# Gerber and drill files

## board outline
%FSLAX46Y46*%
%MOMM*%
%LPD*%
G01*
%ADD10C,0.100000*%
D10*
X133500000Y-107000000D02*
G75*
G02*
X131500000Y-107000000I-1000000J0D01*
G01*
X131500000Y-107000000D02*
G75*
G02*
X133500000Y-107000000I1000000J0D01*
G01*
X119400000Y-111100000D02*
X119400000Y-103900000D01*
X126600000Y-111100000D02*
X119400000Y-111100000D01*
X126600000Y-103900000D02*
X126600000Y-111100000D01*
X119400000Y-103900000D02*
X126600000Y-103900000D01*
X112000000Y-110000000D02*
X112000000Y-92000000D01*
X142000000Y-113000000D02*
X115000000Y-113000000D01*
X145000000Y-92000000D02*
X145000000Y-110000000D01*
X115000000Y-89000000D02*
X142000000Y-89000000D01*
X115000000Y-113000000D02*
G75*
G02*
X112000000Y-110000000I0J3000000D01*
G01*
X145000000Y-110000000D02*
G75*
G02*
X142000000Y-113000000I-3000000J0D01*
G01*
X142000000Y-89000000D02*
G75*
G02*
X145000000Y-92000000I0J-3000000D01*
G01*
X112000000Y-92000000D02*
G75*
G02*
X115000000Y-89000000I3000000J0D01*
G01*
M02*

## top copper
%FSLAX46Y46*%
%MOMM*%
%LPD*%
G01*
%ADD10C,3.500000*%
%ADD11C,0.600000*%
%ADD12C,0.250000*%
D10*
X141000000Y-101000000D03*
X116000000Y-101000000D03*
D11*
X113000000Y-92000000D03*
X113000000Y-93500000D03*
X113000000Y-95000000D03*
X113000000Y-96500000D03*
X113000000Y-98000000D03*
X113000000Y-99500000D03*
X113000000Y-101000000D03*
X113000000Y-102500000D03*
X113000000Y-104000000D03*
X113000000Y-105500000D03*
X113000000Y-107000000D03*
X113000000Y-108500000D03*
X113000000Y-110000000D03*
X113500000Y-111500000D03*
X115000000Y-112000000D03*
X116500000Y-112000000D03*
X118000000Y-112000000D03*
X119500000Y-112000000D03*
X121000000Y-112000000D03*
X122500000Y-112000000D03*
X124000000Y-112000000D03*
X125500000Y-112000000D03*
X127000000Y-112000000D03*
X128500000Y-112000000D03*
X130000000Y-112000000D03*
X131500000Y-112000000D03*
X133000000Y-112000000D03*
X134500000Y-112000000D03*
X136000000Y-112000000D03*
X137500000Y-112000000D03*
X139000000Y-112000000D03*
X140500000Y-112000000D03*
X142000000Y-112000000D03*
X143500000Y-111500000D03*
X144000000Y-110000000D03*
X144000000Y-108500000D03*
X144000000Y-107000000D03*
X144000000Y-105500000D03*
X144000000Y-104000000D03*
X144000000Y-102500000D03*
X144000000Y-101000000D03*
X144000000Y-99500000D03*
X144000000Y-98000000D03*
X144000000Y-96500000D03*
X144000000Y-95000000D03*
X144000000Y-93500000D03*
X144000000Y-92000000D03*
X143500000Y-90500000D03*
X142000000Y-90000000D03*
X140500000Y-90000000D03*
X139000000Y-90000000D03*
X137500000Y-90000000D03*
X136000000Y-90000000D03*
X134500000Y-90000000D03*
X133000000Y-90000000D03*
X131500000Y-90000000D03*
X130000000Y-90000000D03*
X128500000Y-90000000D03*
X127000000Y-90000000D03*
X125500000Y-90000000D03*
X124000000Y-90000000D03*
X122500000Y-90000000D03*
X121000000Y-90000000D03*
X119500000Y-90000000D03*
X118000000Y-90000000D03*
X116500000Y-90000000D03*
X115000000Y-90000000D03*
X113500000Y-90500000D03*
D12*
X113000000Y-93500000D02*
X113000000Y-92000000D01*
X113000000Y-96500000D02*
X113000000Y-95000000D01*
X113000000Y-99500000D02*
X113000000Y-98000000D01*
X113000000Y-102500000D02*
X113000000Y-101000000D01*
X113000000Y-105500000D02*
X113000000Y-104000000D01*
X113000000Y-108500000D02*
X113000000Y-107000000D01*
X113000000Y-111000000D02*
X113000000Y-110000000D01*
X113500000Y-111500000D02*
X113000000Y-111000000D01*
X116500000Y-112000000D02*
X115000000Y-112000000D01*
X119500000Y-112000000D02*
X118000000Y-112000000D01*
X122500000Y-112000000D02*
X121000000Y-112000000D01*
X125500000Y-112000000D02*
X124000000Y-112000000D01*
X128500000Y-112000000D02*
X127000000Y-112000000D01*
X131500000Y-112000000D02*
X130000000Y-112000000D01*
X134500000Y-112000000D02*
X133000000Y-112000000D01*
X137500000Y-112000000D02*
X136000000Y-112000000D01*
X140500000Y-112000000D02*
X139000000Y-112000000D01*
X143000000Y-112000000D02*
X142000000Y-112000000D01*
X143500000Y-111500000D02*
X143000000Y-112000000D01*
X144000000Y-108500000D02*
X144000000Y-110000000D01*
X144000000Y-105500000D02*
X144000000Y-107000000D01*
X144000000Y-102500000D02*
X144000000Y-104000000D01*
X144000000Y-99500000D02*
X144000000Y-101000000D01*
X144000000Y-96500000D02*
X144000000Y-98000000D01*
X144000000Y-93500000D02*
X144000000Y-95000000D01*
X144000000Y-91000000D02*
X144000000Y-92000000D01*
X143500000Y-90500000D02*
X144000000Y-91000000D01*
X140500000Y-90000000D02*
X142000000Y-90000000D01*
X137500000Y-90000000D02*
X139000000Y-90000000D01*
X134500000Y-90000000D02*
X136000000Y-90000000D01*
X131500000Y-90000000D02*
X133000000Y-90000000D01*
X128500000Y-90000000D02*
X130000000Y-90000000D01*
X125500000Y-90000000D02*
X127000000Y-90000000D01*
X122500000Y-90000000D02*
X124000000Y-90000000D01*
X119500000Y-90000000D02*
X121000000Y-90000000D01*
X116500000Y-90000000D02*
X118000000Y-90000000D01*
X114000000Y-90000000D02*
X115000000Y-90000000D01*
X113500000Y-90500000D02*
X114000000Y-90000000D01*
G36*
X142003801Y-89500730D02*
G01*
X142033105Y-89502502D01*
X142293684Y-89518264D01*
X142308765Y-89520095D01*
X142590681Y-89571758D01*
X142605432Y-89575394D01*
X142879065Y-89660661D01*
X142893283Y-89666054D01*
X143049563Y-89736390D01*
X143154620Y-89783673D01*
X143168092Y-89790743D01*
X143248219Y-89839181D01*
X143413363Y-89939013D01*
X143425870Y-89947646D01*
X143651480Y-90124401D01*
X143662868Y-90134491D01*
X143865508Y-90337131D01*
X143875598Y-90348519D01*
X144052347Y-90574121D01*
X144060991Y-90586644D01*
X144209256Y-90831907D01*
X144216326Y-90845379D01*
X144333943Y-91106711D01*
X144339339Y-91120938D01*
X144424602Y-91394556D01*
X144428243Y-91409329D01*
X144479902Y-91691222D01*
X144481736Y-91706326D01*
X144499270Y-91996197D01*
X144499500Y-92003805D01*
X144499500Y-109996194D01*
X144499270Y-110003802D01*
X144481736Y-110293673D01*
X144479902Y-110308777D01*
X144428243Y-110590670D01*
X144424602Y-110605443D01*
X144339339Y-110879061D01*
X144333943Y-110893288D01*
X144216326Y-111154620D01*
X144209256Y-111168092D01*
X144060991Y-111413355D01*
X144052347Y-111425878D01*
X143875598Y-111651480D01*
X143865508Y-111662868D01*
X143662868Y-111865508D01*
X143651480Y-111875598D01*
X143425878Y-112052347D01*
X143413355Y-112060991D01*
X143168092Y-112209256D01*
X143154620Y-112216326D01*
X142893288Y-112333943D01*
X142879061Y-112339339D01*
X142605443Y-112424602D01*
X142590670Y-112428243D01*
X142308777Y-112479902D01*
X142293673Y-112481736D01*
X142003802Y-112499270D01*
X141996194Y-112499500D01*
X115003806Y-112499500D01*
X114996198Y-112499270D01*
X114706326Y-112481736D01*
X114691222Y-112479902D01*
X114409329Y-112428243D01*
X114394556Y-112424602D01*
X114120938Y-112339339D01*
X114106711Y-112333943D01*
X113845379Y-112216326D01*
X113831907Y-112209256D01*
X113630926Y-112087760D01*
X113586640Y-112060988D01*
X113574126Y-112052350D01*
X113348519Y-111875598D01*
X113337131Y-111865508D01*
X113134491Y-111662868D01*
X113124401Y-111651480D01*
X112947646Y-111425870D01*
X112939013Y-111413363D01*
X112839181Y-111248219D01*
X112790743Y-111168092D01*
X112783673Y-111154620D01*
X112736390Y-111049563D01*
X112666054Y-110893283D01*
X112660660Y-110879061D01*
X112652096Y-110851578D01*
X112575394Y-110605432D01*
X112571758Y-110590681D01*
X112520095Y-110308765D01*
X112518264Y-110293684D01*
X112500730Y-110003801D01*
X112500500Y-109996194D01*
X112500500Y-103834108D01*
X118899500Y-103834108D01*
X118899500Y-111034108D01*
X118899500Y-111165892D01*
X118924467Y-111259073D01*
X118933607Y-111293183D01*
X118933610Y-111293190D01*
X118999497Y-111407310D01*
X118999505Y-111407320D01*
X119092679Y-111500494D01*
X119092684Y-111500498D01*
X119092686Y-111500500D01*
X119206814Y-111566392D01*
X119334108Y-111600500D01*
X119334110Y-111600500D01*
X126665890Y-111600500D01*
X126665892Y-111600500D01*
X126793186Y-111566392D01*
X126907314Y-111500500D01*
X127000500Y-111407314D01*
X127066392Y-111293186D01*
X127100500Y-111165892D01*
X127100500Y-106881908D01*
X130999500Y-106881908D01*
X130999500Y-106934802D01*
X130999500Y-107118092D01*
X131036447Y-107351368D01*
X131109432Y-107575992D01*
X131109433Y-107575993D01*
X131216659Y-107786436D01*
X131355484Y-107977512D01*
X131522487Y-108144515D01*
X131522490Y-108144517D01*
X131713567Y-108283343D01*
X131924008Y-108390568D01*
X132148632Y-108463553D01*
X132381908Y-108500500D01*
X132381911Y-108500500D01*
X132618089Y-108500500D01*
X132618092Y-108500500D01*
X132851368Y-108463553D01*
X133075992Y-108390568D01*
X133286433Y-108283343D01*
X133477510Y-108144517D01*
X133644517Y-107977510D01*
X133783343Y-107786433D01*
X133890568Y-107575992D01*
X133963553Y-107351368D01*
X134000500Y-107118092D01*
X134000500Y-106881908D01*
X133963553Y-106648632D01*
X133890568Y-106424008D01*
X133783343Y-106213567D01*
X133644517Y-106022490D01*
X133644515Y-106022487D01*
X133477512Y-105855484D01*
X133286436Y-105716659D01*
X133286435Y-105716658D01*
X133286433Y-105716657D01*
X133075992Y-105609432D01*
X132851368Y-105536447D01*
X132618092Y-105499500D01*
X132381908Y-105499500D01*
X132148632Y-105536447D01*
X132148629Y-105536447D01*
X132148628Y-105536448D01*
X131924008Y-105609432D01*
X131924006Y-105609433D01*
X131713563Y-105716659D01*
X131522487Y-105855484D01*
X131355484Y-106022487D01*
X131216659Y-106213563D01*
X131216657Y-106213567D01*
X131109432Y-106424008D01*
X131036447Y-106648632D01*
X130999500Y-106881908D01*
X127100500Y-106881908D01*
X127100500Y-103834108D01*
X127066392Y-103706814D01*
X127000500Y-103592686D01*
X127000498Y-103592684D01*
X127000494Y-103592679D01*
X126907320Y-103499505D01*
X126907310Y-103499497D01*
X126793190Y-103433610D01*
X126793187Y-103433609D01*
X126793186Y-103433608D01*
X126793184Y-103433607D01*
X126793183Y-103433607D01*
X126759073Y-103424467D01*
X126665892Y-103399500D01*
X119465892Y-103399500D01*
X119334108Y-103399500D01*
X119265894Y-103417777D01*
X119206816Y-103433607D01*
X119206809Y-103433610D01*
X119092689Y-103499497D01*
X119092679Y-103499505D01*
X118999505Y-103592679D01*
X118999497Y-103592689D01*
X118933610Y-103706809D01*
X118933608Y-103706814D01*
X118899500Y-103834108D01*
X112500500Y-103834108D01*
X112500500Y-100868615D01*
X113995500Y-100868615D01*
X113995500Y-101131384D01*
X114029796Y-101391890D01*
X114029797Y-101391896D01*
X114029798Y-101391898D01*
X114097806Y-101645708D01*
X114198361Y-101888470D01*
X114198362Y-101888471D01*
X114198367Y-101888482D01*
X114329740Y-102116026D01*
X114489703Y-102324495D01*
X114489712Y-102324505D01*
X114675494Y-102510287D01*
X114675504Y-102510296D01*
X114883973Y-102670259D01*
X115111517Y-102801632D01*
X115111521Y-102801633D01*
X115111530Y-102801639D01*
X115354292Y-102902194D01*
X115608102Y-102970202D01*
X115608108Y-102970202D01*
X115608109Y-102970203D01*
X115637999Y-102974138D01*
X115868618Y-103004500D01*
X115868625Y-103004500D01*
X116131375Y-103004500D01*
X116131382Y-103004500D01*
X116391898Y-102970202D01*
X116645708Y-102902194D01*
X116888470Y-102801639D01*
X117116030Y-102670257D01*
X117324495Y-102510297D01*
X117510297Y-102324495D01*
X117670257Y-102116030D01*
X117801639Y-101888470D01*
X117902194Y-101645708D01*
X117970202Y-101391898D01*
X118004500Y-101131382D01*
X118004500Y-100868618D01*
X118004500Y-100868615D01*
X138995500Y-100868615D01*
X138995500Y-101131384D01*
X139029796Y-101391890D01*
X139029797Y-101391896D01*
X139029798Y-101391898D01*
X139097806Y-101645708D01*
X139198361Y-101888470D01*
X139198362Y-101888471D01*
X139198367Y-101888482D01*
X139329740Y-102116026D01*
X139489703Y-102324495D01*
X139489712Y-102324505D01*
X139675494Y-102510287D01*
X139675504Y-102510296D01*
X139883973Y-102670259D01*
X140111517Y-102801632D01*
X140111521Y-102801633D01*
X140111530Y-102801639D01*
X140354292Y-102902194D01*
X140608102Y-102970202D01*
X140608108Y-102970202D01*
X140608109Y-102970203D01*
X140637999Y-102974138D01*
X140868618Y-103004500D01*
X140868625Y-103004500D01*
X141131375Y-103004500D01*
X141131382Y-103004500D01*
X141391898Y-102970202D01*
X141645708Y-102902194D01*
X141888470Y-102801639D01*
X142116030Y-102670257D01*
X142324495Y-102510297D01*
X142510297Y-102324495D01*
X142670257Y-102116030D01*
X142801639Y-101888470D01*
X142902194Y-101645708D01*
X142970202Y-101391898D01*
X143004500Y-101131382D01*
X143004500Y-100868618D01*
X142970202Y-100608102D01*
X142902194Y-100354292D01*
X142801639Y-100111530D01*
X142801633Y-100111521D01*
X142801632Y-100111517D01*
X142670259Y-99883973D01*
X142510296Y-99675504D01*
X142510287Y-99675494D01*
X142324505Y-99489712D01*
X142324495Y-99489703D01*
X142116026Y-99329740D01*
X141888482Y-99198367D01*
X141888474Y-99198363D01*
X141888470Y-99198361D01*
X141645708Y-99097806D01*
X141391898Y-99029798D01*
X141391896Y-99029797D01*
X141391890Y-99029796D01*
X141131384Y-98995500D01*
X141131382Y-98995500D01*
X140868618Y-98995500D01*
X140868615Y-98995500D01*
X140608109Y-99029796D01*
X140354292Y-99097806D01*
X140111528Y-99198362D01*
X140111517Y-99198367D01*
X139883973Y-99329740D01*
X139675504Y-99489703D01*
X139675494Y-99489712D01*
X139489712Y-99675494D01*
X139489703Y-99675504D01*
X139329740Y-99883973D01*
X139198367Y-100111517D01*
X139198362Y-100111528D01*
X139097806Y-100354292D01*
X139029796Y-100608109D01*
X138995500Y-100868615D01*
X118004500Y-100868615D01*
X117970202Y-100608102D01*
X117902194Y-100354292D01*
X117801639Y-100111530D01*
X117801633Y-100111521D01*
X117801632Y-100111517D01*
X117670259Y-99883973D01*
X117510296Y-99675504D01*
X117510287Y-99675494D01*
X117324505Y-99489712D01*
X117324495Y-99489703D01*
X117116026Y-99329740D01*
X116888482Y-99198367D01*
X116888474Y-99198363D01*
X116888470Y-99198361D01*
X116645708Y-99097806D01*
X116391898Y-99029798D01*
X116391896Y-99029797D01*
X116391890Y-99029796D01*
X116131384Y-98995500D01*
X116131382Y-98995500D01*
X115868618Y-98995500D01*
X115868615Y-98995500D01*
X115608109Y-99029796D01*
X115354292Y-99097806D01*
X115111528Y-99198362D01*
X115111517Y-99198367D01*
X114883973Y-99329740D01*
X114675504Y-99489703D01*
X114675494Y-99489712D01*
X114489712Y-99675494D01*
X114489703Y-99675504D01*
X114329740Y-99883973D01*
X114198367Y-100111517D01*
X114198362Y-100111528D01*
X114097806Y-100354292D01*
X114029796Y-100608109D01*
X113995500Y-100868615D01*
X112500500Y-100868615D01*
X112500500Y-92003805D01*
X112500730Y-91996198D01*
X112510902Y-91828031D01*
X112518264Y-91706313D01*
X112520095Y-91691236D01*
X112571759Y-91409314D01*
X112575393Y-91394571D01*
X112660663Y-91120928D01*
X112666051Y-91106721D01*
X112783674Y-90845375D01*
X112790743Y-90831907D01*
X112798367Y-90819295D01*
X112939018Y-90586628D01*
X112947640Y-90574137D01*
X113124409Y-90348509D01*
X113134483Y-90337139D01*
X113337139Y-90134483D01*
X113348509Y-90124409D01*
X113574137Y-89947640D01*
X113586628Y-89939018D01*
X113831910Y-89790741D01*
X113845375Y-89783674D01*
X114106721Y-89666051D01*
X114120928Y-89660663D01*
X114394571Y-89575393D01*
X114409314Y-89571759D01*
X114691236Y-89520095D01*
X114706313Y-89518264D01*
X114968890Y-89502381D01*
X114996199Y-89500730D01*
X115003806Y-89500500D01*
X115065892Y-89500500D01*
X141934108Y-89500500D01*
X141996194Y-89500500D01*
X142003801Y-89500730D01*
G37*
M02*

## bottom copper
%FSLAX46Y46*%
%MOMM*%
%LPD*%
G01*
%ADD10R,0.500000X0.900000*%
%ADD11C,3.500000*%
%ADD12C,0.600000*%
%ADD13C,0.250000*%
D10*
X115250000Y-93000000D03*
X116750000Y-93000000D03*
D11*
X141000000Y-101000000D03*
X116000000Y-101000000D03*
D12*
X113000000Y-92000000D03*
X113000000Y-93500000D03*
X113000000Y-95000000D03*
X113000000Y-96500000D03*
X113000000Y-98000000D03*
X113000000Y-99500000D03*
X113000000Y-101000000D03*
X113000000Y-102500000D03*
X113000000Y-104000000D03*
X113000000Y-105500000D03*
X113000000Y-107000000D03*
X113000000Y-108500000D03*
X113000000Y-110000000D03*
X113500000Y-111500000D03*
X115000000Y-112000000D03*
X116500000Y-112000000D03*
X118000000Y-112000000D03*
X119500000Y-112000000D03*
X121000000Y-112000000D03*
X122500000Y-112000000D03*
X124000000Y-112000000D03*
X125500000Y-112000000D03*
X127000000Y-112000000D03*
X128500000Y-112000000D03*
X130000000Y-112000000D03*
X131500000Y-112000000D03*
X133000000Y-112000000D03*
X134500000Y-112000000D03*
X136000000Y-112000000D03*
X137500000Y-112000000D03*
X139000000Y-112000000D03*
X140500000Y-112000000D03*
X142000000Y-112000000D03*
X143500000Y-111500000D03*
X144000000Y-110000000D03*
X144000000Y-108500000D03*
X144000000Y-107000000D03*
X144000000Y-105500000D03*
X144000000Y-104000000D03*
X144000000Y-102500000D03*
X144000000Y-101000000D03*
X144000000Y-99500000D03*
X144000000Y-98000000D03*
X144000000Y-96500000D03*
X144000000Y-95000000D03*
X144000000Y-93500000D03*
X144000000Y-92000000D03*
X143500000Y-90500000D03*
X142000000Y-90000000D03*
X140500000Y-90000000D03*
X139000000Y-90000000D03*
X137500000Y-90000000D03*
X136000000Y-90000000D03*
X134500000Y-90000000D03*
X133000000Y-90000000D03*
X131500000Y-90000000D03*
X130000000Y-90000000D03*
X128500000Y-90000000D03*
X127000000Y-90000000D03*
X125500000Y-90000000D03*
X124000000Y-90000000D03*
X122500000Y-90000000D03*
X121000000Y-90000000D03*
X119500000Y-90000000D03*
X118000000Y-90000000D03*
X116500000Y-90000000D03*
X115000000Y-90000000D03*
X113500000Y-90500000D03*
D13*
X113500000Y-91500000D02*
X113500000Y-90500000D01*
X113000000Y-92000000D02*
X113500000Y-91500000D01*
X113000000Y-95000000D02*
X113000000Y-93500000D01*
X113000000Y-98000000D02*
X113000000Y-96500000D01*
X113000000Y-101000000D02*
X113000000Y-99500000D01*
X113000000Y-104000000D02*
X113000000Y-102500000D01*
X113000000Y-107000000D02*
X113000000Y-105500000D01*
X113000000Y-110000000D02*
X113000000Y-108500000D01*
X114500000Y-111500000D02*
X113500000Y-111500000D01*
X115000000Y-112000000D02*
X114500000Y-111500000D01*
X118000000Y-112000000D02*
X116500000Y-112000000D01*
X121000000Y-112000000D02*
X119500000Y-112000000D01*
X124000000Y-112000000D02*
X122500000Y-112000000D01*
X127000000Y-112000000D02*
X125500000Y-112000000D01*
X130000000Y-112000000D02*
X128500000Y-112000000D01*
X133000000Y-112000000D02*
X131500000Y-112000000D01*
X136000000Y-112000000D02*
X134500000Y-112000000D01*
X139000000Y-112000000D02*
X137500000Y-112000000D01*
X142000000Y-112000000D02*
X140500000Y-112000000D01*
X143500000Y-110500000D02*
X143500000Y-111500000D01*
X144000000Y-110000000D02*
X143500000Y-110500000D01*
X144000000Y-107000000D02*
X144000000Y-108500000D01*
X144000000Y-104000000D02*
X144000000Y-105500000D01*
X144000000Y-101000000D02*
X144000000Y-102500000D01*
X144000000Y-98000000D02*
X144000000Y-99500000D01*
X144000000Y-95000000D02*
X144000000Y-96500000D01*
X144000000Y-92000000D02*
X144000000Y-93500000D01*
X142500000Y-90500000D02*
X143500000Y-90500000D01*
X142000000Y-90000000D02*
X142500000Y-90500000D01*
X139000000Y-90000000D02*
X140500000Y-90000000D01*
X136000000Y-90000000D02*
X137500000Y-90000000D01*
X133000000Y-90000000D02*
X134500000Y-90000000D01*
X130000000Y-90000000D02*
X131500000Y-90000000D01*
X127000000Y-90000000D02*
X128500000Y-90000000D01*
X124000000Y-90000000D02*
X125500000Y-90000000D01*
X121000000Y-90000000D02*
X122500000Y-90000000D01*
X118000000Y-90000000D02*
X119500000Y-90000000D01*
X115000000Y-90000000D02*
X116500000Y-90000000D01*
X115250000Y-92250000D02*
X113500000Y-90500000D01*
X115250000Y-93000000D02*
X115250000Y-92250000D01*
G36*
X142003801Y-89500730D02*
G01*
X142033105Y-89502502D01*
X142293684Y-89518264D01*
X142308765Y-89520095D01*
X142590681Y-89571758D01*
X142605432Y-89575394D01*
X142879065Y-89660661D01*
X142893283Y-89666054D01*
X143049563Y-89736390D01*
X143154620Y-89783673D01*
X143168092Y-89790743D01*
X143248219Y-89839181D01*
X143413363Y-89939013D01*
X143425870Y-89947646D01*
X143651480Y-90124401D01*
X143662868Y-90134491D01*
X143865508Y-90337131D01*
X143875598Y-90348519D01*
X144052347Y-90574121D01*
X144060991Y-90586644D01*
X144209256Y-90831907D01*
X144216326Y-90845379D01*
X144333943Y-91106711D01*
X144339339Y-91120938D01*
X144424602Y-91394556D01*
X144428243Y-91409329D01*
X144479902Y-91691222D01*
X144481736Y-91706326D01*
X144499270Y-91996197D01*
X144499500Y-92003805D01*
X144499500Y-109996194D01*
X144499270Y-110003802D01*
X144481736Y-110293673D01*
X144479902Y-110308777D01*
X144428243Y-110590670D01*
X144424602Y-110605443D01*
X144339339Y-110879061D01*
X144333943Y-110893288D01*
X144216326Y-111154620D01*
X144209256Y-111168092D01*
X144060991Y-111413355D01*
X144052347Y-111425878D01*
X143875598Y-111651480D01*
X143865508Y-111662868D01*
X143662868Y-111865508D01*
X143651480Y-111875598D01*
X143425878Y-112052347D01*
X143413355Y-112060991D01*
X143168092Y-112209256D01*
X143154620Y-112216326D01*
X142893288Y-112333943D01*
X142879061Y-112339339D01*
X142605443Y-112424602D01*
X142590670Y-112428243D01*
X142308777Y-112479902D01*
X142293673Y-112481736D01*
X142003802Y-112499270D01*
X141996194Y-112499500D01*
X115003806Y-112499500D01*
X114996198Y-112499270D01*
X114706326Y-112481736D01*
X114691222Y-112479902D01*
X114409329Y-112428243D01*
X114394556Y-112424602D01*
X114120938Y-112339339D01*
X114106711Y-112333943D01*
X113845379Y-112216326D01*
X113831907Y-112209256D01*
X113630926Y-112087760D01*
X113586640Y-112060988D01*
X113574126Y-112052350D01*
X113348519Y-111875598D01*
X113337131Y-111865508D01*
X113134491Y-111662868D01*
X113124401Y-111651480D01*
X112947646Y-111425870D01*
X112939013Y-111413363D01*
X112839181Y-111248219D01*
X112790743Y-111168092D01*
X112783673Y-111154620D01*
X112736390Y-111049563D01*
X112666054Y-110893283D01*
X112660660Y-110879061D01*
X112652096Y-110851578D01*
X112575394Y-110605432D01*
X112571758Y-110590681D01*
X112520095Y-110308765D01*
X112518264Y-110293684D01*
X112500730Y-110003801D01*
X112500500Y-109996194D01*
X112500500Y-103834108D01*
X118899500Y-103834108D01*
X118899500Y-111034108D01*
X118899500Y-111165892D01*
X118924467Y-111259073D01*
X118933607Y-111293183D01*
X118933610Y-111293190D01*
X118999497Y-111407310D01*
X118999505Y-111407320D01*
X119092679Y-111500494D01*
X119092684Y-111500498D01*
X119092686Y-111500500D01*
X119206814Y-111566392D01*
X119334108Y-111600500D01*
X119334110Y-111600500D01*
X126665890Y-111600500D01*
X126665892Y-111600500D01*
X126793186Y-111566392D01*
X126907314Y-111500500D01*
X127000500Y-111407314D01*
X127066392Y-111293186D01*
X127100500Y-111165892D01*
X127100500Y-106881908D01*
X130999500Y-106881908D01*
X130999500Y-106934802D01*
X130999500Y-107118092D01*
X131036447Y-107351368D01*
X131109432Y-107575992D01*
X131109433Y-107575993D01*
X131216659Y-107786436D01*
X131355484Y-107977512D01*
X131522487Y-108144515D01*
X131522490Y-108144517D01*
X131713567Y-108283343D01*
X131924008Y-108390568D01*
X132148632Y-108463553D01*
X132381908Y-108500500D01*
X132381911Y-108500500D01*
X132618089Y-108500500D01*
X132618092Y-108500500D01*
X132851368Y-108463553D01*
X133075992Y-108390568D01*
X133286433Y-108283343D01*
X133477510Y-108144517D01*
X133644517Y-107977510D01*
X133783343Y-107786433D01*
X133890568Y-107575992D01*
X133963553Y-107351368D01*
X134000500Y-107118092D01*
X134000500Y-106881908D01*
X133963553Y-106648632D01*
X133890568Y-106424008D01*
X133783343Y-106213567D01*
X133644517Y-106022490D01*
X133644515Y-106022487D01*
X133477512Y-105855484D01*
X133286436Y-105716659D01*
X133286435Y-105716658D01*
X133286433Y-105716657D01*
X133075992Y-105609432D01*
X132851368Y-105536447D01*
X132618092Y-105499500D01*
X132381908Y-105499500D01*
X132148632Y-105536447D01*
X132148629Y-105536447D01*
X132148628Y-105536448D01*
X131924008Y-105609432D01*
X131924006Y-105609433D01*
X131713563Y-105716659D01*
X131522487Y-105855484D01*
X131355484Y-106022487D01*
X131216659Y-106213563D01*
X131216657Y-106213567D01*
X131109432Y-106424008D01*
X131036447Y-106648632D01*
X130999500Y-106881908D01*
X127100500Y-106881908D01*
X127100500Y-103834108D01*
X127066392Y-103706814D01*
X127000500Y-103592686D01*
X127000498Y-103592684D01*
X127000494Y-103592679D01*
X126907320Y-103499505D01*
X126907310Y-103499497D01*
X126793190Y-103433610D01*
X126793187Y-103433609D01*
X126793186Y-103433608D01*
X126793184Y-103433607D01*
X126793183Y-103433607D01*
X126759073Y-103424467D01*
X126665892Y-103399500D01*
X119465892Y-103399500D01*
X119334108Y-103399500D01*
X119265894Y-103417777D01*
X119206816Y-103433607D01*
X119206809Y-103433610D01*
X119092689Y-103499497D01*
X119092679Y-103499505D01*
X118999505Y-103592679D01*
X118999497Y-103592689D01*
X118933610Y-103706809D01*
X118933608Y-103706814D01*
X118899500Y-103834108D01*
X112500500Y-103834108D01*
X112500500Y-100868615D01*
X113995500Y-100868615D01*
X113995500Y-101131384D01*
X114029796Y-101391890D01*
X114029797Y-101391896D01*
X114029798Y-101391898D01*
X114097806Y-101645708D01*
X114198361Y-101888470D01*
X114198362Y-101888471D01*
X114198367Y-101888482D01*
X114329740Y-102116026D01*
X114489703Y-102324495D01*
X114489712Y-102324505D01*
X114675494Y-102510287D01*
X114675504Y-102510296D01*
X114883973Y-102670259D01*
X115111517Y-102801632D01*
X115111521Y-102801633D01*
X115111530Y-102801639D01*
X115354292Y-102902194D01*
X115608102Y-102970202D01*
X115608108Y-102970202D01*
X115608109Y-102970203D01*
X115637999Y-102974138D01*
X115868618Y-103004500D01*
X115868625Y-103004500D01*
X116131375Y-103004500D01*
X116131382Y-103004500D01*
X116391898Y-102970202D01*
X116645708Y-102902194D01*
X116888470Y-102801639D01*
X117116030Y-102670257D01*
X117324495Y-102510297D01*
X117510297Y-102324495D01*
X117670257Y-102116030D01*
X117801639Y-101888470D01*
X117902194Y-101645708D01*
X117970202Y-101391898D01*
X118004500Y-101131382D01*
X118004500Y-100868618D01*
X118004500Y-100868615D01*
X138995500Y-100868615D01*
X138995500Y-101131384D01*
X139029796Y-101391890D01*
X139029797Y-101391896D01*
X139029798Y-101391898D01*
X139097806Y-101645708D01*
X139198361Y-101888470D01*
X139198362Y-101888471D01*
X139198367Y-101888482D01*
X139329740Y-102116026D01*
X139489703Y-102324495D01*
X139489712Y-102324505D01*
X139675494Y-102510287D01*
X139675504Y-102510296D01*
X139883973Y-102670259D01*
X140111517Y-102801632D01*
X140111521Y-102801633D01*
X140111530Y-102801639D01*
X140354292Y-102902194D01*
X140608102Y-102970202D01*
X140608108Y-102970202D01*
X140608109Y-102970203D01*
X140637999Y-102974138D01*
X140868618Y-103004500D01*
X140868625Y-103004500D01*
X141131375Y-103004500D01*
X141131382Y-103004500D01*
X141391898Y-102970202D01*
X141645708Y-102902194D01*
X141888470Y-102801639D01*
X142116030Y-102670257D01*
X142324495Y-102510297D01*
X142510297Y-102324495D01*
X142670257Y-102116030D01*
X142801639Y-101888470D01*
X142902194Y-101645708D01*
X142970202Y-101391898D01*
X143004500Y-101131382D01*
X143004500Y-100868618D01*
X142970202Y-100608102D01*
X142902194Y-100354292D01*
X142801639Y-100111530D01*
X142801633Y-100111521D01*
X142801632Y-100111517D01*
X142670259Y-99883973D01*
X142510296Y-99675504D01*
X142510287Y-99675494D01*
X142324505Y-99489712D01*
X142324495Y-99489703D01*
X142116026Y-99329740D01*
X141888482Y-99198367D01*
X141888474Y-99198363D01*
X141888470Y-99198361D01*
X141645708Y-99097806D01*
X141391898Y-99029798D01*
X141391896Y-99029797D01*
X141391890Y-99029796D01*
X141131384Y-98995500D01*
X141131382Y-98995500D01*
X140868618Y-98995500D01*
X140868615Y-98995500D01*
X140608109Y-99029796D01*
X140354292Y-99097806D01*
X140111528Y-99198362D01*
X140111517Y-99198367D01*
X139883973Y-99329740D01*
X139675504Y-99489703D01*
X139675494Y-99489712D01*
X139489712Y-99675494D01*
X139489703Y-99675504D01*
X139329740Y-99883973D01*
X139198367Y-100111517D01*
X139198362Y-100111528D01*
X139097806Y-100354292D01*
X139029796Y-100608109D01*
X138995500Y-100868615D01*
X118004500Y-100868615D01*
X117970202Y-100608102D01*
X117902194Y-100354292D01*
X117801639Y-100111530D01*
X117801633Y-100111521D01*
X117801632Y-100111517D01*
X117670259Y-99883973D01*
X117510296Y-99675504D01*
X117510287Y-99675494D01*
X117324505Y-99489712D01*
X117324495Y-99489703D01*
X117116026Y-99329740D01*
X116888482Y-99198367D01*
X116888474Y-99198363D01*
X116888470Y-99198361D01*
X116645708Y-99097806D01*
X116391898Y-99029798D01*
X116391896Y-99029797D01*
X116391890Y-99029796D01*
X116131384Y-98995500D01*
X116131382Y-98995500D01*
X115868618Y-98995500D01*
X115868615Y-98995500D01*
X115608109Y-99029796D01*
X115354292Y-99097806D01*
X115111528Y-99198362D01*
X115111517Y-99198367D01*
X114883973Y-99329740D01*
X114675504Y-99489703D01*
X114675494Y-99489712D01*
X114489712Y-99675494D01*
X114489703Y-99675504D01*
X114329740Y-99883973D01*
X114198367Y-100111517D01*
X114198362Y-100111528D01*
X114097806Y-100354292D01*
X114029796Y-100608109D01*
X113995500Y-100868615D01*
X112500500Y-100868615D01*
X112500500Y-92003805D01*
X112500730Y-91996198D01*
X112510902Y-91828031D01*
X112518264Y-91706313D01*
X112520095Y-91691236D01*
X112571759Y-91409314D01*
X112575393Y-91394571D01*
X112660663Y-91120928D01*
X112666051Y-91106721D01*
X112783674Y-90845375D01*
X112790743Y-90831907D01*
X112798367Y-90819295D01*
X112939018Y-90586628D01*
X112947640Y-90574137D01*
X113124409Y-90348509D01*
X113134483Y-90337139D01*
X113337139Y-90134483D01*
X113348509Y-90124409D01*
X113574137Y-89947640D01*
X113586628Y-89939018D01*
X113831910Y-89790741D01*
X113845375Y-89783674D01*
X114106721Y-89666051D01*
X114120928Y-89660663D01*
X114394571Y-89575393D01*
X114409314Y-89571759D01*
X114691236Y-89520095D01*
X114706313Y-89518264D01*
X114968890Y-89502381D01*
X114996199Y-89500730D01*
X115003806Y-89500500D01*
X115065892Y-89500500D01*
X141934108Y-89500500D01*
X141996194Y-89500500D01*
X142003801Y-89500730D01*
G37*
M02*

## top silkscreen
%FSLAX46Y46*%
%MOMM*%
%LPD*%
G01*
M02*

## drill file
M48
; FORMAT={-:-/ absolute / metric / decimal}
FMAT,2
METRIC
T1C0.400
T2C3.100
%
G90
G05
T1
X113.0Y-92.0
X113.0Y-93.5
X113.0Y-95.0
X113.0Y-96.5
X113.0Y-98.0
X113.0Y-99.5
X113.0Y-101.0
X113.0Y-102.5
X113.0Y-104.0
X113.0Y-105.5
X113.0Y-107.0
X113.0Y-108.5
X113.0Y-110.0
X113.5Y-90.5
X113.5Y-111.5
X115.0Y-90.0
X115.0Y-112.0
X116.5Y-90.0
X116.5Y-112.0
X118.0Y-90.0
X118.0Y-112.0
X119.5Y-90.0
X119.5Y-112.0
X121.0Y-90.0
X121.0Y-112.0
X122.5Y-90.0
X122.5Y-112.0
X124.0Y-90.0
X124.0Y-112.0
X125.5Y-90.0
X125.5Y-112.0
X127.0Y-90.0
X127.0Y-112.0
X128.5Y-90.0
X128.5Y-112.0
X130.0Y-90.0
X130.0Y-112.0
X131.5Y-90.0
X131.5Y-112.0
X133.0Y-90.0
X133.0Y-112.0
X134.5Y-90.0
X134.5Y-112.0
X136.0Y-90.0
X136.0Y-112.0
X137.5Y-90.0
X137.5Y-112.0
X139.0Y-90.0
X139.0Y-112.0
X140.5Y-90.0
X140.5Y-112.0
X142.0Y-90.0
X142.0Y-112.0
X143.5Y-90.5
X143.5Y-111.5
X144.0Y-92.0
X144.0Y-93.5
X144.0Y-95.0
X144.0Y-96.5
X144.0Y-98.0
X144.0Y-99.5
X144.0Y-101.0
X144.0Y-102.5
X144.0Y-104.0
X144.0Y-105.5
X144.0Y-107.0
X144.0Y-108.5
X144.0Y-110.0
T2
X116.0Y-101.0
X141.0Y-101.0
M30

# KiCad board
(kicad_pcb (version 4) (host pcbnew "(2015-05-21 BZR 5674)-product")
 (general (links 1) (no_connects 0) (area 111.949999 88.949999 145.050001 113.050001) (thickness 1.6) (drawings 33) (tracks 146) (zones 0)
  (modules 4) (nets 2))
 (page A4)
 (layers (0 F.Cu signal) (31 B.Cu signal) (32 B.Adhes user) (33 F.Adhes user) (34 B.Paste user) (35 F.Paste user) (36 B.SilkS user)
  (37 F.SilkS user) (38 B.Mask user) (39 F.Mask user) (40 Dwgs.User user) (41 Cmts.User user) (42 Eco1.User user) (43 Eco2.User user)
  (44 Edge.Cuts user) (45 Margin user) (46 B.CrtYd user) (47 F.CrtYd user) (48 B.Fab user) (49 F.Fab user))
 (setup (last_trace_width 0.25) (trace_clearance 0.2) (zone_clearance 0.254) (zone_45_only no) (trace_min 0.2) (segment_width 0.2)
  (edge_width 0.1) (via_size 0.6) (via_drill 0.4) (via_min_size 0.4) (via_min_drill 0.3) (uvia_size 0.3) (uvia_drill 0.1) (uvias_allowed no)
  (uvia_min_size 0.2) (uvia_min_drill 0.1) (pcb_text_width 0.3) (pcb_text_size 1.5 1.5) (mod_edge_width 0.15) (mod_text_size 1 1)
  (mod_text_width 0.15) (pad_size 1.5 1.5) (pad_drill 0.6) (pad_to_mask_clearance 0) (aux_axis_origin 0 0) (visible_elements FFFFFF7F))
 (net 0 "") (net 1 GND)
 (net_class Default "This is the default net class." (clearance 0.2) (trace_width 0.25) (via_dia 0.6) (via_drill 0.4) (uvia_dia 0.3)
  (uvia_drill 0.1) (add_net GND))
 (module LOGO (layer F.Cu) (at 123 95.25)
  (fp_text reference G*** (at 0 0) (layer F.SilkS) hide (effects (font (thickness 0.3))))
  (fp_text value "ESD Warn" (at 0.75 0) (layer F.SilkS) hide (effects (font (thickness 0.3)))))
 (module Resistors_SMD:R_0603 (layer B.Cu) (at 116 93) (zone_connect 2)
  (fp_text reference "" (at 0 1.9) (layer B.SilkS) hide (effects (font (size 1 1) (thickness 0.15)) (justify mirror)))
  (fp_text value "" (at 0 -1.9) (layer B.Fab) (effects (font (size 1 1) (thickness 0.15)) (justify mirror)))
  (pad 1 smd rect (at -0.75 0) (size 0.5 0.9) (layers B.Cu B.Paste B.Mask) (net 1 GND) (zone_connect 2))
  (pad 2 smd rect (at 0.75 0) (size 0.5 0.9) (layers B.Cu B.Paste B.Mask) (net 1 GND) (zone_connect 2)))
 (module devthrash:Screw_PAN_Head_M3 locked (layer B.Cu) (at 141 101)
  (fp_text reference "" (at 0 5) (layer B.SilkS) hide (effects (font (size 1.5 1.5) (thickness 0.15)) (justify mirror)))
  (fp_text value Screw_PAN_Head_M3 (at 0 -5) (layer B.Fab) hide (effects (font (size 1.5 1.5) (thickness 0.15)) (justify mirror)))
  (pad "" np_thru_hole circle (at 0 0) (size 3.5 3.5) (drill 3.1) (layers *.Cu *.Mask B.SilkS)))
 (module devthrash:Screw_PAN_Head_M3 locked (layer B.Cu) (at 116 101)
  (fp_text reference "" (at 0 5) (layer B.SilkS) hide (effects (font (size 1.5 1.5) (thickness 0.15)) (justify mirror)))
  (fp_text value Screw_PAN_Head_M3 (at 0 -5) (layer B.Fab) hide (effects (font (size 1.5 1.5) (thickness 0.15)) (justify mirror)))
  (pad "" np_thru_hole circle (at 0 0) (size 3.5 3.5) (drill 3.1) (layers *.Cu *.Mask B.SilkS)))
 (gr_circle (center 132.5 107) (end 133.5 107) (layer Edge.Cuts) (width 0.1))
 (gr_line (start 119.4 111.1) (end 119.4 103.9) (angle 90) (layer Edge.Cuts) (width 0.1))
 (gr_line (start 126.6 111.1) (end 119.4 111.1) (angle 90) (layer Edge.Cuts) (width 0.1))
 (gr_line (start 126.6 103.9) (end 126.6 111.1) (angle 90) (layer Edge.Cuts) (width 0.1))
 (gr_line (start 119.4 103.9) (end 126.6 103.9) (angle 90) (layer Edge.Cuts) (width 0.1))
 (gr_line (start 112 110) (end 112 92) (angle 90) (layer Edge.Cuts) (width 0.1))
 (gr_line (start 142 113) (end 115 113) (angle 90) (layer Edge.Cuts) (width 0.1))
 (gr_line (start 145 92) (end 145 110) (angle 90) (layer Edge.Cuts) (width 0.1))
 (gr_line (start 115 89) (end 142 89) (angle 90) (layer Edge.Cuts) (width 0.1))
 (gr_arc (start 115 110) (end 115 113) (angle 90) (layer Edge.Cuts) (width 0.1))
 (gr_arc (start 142 110) (end 145 110) (angle 90) (layer Edge.Cuts) (width 0.1))
 (gr_arc (start 142 92) (end 142 89) (angle 90) (layer Edge.Cuts) (width 0.1))
 (gr_arc (start 115 92) (end 112 92) (angle 90) (layer Edge.Cuts) (width 0.1))
 (segment (start 113.5 91.5) (end 113.5 90.5) (width 0.25) (layer B.Cu) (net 1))
 (segment (start 113 92) (end 113.5 91.5) (width 0.25) (layer B.Cu) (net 1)) (via (at 113 92) (size 0.6) (layers F.Cu B.Cu) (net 1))
 (segment (start 113 93.5) (end 113 92) (width 0.25) (layer F.Cu) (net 1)) (via (at 113 93.5) (size 0.6) (layers F.Cu B.Cu) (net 1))
 (segment (start 113 95) (end 113 93.5) (width 0.25) (layer B.Cu) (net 1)) (via (at 113 95) (size 0.6) (layers F.Cu B.Cu) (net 1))
 (segment (start 113 96.5) (end 113 95) (width 0.25) (layer F.Cu) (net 1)) (via (at 113 96.5) (size 0.6) (layers F.Cu B.Cu) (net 1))
 (segment (start 113 98) (end 113 96.5) (width 0.25) (layer B.Cu) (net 1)) (via (at 113 98) (size 0.6) (layers F.Cu B.Cu) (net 1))
 (segment (start 113 99.5) (end 113 98) (width 0.25) (layer F.Cu) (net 1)) (via (at 113 99.5) (size 0.6) (layers F.Cu B.Cu) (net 1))
 (segment (start 113 101) (end 113 99.5) (width 0.25) (layer B.Cu) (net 1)) (via (at 113 101) (size 0.6) (layers F.Cu B.Cu) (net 1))
 (segment (start 113 102.5) (end 113 101) (width 0.25) (layer F.Cu) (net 1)) (via (at 113 102.5) (size 0.6) (layers F.Cu B.Cu) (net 1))
 (segment (start 113 104) (end 113 102.5) (width 0.25) (layer B.Cu) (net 1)) (via (at 113 104) (size 0.6) (layers F.Cu B.Cu) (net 1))
 (segment (start 113 105.5) (end 113 104) (width 0.25) (layer F.Cu) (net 1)) (via (at 113 105.5) (size 0.6) (layers F.Cu B.Cu) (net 1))
 (segment (start 113 107) (end 113 105.5) (width 0.25) (layer B.Cu) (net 1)) (via (at 113 107) (size 0.6) (layers F.Cu B.Cu) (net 1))
 (segment (start 113 108.5) (end 113 107) (width 0.25) (layer F.Cu) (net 1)) (via (at 113 108.5) (size 0.6) (layers F.Cu B.Cu) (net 1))
 (segment (start 113 110) (end 113 108.5) (width 0.25) (layer B.Cu) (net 1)) (via (at 113 110) (size 0.6) (layers F.Cu B.Cu) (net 1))
 (segment (start 113 111) (end 113 110) (width 0.25) (layer F.Cu) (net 1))
 (segment (start 113.5 111.5) (end 113 111) (width 0.25) (layer F.Cu) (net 1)) (via (at 113.5 111.5) (size 0.6) (layers F.Cu B.Cu) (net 1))
 (segment (start 114.5 111.5) (end 113.5 111.5) (width 0.25) (layer B.Cu) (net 1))
 (segment (start 115 112) (end 114.5 111.5) (width 0.25) (layer B.Cu) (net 1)) (via (at 115 112) (size 0.6) (layers F.Cu B.Cu) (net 1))
 (segment (start 116.5 112) (end 115 112) (width 0.25) (layer F.Cu) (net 1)) (via (at 116.5 112) (size 0.6) (layers F.Cu B.Cu) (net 1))
 (segment (start 118 112) (end 116.5 112) (width 0.25) (layer B.Cu) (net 1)) (via (at 118 112) (size 0.6) (layers F.Cu B.Cu) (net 1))
 (segment (start 119.5 112) (end 118 112) (width 0.25) (layer F.Cu) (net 1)) (via (at 119.5 112) (size 0.6) (layers F.Cu B.Cu) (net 1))
 (segment (start 121 112) (end 119.5 112) (width 0.25) (layer B.Cu) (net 1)) (via (at 121 112) (size 0.6) (layers F.Cu B.Cu) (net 1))
 (segment (start 122.5 112) (end 121 112) (width 0.25) (layer F.Cu) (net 1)) (via (at 122.5 112) (size 0.6) (layers F.Cu B.Cu) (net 1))
 (segment (start 124 112) (end 122.5 112) (width 0.25) (layer B.Cu) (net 1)) (via (at 124 112) (size 0.6) (layers F.Cu B.Cu) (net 1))
 (segment (start 125.5 112) (end 124 112) (width 0.25) (layer F.Cu) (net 1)) (via (at 125.5 112) (size 0.6) (layers F.Cu B.Cu) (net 1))
 (segment (start 127 112) (end 125.5 112) (width 0.25) (layer B.Cu) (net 1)) (via (at 127 112) (size 0.6) (layers F.Cu B.Cu) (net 1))
 (segment (start 128.5 112) (end 127 112) (width 0.25) (layer F.Cu) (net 1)) (via (at 128.5 112) (size 0.6) (layers F.Cu B.Cu) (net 1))
 (segment (start 130 112) (end 128.5 112) (width 0.25) (layer B.Cu) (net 1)) (via (at 130 112) (size 0.6) (layers F.Cu B.Cu) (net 1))
 (segment (start 131.5 112) (end 130 112) (width 0.25) (layer F.Cu) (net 1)) (via (at 131.5 112) (size 0.6) (layers F.Cu B.Cu) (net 1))
 (segment (start 133 112) (end 131.5 112) (width 0.25) (layer B.Cu) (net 1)) (via (at 133 112) (size 0.6) (layers F.Cu B.Cu) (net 1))
 (segment (start 134.5 112) (end 133 112) (width 0.25) (layer F.Cu) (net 1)) (via (at 134.5 112) (size 0.6) (layers F.Cu B.Cu) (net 1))
 (segment (start 136 112) (end 134.5 112) (width 0.25) (layer B.Cu) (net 1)) (via (at 136 112) (size 0.6) (layers F.Cu B.Cu) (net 1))
 (segment (start 137.5 112) (end 136 112) (width 0.25) (layer F.Cu) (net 1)) (via (at 137.5 112) (size 0.6) (layers F.Cu B.Cu) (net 1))
 (segment (start 139 112) (end 137.5 112) (width 0.25) (layer B.Cu) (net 1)) (via (at 139 112) (size 0.6) (layers F.Cu B.Cu) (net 1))
 (segment (start 140.5 112) (end 139 112) (width 0.25) (layer F.Cu) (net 1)) (via (at 140.5 112) (size 0.6) (layers F.Cu B.Cu) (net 1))
 (segment (start 142 112) (end 140.5 112) (width 0.25) (layer B.Cu) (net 1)) (via (at 142 112) (size 0.6) (layers F.Cu B.Cu) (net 1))
 (segment (start 143 112) (end 142 112) (width 0.25) (layer F.Cu) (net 1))
 (segment (start 143.5 111.5) (end 143 112) (width 0.25) (layer F.Cu) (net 1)) (via (at 143.5 111.5) (size 0.6) (layers F.Cu B.Cu) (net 1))
 (segment (start 143.5 110.5) (end 143.5 111.5) (width 0.25) (layer B.Cu) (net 1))
 (segment (start 144 110) (end 143.5 110.5) (width 0.25) (layer B.Cu) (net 1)) (via (at 144 110) (size 0.6) (layers F.Cu B.Cu) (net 1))
 (segment (start 144 108.5) (end 144 110) (width 0.25) (layer F.Cu) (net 1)) (via (at 144 108.5) (size 0.6) (layers F.Cu B.Cu) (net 1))
 (segment (start 144 107) (end 144 108.5) (width 0.25) (layer B.Cu) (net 1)) (via (at 144 107) (size 0.6) (layers F.Cu B.Cu) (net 1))
 (segment (start 144 105.5) (end 144 107) (width 0.25) (layer F.Cu) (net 1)) (via (at 144 105.5) (size 0.6) (layers F.Cu B.Cu) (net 1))
 (segment (start 144 104) (end 144 105.5) (width 0.25) (layer B.Cu) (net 1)) (via (at 144 104) (size 0.6) (layers F.Cu B.Cu) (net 1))
 (segment (start 144 102.5) (end 144 104) (width 0.25) (layer F.Cu) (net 1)) (via (at 144 102.5) (size 0.6) (layers F.Cu B.Cu) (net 1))
 (segment (start 144 101) (end 144 102.5) (width 0.25) (layer B.Cu) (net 1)) (via (at 144 101) (size 0.6) (layers F.Cu B.Cu) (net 1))
 (segment (start 144 99.5) (end 144 101) (width 0.25) (layer F.Cu) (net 1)) (via (at 144 99.5) (size 0.6) (layers F.Cu B.Cu) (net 1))
 (segment (start 144 98) (end 144 99.5) (width 0.25) (layer B.Cu) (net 1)) (via (at 144 98) (size 0.6) (layers F.Cu B.Cu) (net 1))
 (segment (start 144 96.5) (end 144 98) (width 0.25) (layer F.Cu) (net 1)) (via (at 144 96.5) (size 0.6) (layers F.Cu B.Cu) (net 1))
 (segment (start 144 95) (end 144 96.5) (width 0.25) (layer B.Cu) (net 1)) (via (at 144 95) (size 0.6) (layers F.Cu B.Cu) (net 1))
 (segment (start 144 93.5) (end 144 95) (width 0.25) (layer F.Cu) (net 1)) (via (at 144 93.5) (size 0.6) (layers F.Cu B.Cu) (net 1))
 (segment (start 144 92) (end 144 93.5) (width 0.25) (layer B.Cu) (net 1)) (via (at 144 92) (size 0.6) (layers F.Cu B.Cu) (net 1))
 (segment (start 144 91) (end 144 92) (width 0.25) (layer F.Cu) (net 1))
 (segment (start 143.5 90.5) (end 144 91) (width 0.25) (layer F.Cu) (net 1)) (via (at 143.5 90.5) (size 0.6) (layers F.Cu B.Cu) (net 1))
 (segment (start 142.5 90.5) (end 143.5 90.5) (width 0.25) (layer B.Cu) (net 1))
 (segment (start 142 90) (end 142.5 90.5) (width 0.25) (layer B.Cu) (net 1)) (via (at 142 90) (size 0.6) (layers F.Cu B.Cu) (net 1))
 (segment (start 140.5 90) (end 142 90) (width 0.25) (layer F.Cu) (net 1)) (via (at 140.5 90) (size 0.6) (layers F.Cu B.Cu) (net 1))
 (segment (start 139 90) (end 140.5 90) (width 0.25) (layer B.Cu) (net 1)) (via (at 139 90) (size 0.6) (layers F.Cu B.Cu) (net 1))
 (segment (start 137.5 90) (end 139 90) (width 0.25) (layer F.Cu) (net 1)) (via (at 137.5 90) (size 0.6) (layers F.Cu B.Cu) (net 1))
 (segment (start 136 90) (end 137.5 90) (width 0.25) (layer B.Cu) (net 1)) (via (at 136 90) (size 0.6) (layers F.Cu B.Cu) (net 1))
 (segment (start 134.5 90) (end 136 90) (width 0.25) (layer F.Cu) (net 1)) (via (at 134.5 90) (size 0.6) (layers F.Cu B.Cu) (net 1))
 (segment (start 133 90) (end 134.5 90) (width 0.25) (layer B.Cu) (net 1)) (via (at 133 90) (size 0.6) (layers F.Cu B.Cu) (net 1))
 (segment (start 131.5 90) (end 133 90) (width 0.25) (layer F.Cu) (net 1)) (via (at 131.5 90) (size 0.6) (layers F.Cu B.Cu) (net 1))
 (segment (start 130 90) (end 131.5 90) (width 0.25) (layer B.Cu) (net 1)) (via (at 130 90) (size 0.6) (layers F.Cu B.Cu) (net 1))
 (segment (start 128.5 90) (end 130 90) (width 0.25) (layer F.Cu) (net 1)) (via (at 128.5 90) (size 0.6) (layers F.Cu B.Cu) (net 1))
 (segment (start 127 90) (end 128.5 90) (width 0.25) (layer B.Cu) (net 1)) (via (at 127 90) (size 0.6) (layers F.Cu B.Cu) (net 1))
 (segment (start 125.5 90) (end 127 90) (width 0.25) (layer F.Cu) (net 1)) (via (at 125.5 90) (size 0.6) (layers F.Cu B.Cu) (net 1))
 (segment (start 124 90) (end 125.5 90) (width 0.25) (layer B.Cu) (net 1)) (via (at 124 90) (size 0.6) (layers F.Cu B.Cu) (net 1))
 (segment (start 122.5 90) (end 124 90) (width 0.25) (layer F.Cu) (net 1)) (via (at 122.5 90) (size 0.6) (layers F.Cu B.Cu) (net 1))
 (segment (start 121 90) (end 122.5 90) (width 0.25) (layer B.Cu) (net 1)) (via (at 121 90) (size 0.6) (layers F.Cu B.Cu) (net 1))
 (segment (start 119.5 90) (end 121 90) (width 0.25) (layer F.Cu) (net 1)) (via (at 119.5 90) (size 0.6) (layers F.Cu B.Cu) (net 1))
 (segment (start 118 90) (end 119.5 90) (width 0.25) (layer B.Cu) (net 1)) (via (at 118 90) (size 0.6) (layers F.Cu B.Cu) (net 1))
 (segment (start 116.5 90) (end 118 90) (width 0.25) (layer F.Cu) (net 1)) (via (at 116.5 90) (size 0.6) (layers F.Cu B.Cu) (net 1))
 (segment (start 115 90) (end 116.5 90) (width 0.25) (layer B.Cu) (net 1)) (via (at 115 90) (size 0.6) (layers F.Cu B.Cu) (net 1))
 (segment (start 114 90) (end 115 90) (width 0.25) (layer F.Cu) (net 1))
 (segment (start 113.5 90.5) (end 114 90) (width 0.25) (layer F.Cu) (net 1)) (via (at 113.5 90.5) (size 0.6) (layers F.Cu B.Cu) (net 1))
 (segment (start 115.25 92.25) (end 113.5 90.5) (width 0.25) (layer B.Cu) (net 1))
 (segment (start 115.25 93) (end 115.25 92.25) (width 0.25) (layer B.Cu) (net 1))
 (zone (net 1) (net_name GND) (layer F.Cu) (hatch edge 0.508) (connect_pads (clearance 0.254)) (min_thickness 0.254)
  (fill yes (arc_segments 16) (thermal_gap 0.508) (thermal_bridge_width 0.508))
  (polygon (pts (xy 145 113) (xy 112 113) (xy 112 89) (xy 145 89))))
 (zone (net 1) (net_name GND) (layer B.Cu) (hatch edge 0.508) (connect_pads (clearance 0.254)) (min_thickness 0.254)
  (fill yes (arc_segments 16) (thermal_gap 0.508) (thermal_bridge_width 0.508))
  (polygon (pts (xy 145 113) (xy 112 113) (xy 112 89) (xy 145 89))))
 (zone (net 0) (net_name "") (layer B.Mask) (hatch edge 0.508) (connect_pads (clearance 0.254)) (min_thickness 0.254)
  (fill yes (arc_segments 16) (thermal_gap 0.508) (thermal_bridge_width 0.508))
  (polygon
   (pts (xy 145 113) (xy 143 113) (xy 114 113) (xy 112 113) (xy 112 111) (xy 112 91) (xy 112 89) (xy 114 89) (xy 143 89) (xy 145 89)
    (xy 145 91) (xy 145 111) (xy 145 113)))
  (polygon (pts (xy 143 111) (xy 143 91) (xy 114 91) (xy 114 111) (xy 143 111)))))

